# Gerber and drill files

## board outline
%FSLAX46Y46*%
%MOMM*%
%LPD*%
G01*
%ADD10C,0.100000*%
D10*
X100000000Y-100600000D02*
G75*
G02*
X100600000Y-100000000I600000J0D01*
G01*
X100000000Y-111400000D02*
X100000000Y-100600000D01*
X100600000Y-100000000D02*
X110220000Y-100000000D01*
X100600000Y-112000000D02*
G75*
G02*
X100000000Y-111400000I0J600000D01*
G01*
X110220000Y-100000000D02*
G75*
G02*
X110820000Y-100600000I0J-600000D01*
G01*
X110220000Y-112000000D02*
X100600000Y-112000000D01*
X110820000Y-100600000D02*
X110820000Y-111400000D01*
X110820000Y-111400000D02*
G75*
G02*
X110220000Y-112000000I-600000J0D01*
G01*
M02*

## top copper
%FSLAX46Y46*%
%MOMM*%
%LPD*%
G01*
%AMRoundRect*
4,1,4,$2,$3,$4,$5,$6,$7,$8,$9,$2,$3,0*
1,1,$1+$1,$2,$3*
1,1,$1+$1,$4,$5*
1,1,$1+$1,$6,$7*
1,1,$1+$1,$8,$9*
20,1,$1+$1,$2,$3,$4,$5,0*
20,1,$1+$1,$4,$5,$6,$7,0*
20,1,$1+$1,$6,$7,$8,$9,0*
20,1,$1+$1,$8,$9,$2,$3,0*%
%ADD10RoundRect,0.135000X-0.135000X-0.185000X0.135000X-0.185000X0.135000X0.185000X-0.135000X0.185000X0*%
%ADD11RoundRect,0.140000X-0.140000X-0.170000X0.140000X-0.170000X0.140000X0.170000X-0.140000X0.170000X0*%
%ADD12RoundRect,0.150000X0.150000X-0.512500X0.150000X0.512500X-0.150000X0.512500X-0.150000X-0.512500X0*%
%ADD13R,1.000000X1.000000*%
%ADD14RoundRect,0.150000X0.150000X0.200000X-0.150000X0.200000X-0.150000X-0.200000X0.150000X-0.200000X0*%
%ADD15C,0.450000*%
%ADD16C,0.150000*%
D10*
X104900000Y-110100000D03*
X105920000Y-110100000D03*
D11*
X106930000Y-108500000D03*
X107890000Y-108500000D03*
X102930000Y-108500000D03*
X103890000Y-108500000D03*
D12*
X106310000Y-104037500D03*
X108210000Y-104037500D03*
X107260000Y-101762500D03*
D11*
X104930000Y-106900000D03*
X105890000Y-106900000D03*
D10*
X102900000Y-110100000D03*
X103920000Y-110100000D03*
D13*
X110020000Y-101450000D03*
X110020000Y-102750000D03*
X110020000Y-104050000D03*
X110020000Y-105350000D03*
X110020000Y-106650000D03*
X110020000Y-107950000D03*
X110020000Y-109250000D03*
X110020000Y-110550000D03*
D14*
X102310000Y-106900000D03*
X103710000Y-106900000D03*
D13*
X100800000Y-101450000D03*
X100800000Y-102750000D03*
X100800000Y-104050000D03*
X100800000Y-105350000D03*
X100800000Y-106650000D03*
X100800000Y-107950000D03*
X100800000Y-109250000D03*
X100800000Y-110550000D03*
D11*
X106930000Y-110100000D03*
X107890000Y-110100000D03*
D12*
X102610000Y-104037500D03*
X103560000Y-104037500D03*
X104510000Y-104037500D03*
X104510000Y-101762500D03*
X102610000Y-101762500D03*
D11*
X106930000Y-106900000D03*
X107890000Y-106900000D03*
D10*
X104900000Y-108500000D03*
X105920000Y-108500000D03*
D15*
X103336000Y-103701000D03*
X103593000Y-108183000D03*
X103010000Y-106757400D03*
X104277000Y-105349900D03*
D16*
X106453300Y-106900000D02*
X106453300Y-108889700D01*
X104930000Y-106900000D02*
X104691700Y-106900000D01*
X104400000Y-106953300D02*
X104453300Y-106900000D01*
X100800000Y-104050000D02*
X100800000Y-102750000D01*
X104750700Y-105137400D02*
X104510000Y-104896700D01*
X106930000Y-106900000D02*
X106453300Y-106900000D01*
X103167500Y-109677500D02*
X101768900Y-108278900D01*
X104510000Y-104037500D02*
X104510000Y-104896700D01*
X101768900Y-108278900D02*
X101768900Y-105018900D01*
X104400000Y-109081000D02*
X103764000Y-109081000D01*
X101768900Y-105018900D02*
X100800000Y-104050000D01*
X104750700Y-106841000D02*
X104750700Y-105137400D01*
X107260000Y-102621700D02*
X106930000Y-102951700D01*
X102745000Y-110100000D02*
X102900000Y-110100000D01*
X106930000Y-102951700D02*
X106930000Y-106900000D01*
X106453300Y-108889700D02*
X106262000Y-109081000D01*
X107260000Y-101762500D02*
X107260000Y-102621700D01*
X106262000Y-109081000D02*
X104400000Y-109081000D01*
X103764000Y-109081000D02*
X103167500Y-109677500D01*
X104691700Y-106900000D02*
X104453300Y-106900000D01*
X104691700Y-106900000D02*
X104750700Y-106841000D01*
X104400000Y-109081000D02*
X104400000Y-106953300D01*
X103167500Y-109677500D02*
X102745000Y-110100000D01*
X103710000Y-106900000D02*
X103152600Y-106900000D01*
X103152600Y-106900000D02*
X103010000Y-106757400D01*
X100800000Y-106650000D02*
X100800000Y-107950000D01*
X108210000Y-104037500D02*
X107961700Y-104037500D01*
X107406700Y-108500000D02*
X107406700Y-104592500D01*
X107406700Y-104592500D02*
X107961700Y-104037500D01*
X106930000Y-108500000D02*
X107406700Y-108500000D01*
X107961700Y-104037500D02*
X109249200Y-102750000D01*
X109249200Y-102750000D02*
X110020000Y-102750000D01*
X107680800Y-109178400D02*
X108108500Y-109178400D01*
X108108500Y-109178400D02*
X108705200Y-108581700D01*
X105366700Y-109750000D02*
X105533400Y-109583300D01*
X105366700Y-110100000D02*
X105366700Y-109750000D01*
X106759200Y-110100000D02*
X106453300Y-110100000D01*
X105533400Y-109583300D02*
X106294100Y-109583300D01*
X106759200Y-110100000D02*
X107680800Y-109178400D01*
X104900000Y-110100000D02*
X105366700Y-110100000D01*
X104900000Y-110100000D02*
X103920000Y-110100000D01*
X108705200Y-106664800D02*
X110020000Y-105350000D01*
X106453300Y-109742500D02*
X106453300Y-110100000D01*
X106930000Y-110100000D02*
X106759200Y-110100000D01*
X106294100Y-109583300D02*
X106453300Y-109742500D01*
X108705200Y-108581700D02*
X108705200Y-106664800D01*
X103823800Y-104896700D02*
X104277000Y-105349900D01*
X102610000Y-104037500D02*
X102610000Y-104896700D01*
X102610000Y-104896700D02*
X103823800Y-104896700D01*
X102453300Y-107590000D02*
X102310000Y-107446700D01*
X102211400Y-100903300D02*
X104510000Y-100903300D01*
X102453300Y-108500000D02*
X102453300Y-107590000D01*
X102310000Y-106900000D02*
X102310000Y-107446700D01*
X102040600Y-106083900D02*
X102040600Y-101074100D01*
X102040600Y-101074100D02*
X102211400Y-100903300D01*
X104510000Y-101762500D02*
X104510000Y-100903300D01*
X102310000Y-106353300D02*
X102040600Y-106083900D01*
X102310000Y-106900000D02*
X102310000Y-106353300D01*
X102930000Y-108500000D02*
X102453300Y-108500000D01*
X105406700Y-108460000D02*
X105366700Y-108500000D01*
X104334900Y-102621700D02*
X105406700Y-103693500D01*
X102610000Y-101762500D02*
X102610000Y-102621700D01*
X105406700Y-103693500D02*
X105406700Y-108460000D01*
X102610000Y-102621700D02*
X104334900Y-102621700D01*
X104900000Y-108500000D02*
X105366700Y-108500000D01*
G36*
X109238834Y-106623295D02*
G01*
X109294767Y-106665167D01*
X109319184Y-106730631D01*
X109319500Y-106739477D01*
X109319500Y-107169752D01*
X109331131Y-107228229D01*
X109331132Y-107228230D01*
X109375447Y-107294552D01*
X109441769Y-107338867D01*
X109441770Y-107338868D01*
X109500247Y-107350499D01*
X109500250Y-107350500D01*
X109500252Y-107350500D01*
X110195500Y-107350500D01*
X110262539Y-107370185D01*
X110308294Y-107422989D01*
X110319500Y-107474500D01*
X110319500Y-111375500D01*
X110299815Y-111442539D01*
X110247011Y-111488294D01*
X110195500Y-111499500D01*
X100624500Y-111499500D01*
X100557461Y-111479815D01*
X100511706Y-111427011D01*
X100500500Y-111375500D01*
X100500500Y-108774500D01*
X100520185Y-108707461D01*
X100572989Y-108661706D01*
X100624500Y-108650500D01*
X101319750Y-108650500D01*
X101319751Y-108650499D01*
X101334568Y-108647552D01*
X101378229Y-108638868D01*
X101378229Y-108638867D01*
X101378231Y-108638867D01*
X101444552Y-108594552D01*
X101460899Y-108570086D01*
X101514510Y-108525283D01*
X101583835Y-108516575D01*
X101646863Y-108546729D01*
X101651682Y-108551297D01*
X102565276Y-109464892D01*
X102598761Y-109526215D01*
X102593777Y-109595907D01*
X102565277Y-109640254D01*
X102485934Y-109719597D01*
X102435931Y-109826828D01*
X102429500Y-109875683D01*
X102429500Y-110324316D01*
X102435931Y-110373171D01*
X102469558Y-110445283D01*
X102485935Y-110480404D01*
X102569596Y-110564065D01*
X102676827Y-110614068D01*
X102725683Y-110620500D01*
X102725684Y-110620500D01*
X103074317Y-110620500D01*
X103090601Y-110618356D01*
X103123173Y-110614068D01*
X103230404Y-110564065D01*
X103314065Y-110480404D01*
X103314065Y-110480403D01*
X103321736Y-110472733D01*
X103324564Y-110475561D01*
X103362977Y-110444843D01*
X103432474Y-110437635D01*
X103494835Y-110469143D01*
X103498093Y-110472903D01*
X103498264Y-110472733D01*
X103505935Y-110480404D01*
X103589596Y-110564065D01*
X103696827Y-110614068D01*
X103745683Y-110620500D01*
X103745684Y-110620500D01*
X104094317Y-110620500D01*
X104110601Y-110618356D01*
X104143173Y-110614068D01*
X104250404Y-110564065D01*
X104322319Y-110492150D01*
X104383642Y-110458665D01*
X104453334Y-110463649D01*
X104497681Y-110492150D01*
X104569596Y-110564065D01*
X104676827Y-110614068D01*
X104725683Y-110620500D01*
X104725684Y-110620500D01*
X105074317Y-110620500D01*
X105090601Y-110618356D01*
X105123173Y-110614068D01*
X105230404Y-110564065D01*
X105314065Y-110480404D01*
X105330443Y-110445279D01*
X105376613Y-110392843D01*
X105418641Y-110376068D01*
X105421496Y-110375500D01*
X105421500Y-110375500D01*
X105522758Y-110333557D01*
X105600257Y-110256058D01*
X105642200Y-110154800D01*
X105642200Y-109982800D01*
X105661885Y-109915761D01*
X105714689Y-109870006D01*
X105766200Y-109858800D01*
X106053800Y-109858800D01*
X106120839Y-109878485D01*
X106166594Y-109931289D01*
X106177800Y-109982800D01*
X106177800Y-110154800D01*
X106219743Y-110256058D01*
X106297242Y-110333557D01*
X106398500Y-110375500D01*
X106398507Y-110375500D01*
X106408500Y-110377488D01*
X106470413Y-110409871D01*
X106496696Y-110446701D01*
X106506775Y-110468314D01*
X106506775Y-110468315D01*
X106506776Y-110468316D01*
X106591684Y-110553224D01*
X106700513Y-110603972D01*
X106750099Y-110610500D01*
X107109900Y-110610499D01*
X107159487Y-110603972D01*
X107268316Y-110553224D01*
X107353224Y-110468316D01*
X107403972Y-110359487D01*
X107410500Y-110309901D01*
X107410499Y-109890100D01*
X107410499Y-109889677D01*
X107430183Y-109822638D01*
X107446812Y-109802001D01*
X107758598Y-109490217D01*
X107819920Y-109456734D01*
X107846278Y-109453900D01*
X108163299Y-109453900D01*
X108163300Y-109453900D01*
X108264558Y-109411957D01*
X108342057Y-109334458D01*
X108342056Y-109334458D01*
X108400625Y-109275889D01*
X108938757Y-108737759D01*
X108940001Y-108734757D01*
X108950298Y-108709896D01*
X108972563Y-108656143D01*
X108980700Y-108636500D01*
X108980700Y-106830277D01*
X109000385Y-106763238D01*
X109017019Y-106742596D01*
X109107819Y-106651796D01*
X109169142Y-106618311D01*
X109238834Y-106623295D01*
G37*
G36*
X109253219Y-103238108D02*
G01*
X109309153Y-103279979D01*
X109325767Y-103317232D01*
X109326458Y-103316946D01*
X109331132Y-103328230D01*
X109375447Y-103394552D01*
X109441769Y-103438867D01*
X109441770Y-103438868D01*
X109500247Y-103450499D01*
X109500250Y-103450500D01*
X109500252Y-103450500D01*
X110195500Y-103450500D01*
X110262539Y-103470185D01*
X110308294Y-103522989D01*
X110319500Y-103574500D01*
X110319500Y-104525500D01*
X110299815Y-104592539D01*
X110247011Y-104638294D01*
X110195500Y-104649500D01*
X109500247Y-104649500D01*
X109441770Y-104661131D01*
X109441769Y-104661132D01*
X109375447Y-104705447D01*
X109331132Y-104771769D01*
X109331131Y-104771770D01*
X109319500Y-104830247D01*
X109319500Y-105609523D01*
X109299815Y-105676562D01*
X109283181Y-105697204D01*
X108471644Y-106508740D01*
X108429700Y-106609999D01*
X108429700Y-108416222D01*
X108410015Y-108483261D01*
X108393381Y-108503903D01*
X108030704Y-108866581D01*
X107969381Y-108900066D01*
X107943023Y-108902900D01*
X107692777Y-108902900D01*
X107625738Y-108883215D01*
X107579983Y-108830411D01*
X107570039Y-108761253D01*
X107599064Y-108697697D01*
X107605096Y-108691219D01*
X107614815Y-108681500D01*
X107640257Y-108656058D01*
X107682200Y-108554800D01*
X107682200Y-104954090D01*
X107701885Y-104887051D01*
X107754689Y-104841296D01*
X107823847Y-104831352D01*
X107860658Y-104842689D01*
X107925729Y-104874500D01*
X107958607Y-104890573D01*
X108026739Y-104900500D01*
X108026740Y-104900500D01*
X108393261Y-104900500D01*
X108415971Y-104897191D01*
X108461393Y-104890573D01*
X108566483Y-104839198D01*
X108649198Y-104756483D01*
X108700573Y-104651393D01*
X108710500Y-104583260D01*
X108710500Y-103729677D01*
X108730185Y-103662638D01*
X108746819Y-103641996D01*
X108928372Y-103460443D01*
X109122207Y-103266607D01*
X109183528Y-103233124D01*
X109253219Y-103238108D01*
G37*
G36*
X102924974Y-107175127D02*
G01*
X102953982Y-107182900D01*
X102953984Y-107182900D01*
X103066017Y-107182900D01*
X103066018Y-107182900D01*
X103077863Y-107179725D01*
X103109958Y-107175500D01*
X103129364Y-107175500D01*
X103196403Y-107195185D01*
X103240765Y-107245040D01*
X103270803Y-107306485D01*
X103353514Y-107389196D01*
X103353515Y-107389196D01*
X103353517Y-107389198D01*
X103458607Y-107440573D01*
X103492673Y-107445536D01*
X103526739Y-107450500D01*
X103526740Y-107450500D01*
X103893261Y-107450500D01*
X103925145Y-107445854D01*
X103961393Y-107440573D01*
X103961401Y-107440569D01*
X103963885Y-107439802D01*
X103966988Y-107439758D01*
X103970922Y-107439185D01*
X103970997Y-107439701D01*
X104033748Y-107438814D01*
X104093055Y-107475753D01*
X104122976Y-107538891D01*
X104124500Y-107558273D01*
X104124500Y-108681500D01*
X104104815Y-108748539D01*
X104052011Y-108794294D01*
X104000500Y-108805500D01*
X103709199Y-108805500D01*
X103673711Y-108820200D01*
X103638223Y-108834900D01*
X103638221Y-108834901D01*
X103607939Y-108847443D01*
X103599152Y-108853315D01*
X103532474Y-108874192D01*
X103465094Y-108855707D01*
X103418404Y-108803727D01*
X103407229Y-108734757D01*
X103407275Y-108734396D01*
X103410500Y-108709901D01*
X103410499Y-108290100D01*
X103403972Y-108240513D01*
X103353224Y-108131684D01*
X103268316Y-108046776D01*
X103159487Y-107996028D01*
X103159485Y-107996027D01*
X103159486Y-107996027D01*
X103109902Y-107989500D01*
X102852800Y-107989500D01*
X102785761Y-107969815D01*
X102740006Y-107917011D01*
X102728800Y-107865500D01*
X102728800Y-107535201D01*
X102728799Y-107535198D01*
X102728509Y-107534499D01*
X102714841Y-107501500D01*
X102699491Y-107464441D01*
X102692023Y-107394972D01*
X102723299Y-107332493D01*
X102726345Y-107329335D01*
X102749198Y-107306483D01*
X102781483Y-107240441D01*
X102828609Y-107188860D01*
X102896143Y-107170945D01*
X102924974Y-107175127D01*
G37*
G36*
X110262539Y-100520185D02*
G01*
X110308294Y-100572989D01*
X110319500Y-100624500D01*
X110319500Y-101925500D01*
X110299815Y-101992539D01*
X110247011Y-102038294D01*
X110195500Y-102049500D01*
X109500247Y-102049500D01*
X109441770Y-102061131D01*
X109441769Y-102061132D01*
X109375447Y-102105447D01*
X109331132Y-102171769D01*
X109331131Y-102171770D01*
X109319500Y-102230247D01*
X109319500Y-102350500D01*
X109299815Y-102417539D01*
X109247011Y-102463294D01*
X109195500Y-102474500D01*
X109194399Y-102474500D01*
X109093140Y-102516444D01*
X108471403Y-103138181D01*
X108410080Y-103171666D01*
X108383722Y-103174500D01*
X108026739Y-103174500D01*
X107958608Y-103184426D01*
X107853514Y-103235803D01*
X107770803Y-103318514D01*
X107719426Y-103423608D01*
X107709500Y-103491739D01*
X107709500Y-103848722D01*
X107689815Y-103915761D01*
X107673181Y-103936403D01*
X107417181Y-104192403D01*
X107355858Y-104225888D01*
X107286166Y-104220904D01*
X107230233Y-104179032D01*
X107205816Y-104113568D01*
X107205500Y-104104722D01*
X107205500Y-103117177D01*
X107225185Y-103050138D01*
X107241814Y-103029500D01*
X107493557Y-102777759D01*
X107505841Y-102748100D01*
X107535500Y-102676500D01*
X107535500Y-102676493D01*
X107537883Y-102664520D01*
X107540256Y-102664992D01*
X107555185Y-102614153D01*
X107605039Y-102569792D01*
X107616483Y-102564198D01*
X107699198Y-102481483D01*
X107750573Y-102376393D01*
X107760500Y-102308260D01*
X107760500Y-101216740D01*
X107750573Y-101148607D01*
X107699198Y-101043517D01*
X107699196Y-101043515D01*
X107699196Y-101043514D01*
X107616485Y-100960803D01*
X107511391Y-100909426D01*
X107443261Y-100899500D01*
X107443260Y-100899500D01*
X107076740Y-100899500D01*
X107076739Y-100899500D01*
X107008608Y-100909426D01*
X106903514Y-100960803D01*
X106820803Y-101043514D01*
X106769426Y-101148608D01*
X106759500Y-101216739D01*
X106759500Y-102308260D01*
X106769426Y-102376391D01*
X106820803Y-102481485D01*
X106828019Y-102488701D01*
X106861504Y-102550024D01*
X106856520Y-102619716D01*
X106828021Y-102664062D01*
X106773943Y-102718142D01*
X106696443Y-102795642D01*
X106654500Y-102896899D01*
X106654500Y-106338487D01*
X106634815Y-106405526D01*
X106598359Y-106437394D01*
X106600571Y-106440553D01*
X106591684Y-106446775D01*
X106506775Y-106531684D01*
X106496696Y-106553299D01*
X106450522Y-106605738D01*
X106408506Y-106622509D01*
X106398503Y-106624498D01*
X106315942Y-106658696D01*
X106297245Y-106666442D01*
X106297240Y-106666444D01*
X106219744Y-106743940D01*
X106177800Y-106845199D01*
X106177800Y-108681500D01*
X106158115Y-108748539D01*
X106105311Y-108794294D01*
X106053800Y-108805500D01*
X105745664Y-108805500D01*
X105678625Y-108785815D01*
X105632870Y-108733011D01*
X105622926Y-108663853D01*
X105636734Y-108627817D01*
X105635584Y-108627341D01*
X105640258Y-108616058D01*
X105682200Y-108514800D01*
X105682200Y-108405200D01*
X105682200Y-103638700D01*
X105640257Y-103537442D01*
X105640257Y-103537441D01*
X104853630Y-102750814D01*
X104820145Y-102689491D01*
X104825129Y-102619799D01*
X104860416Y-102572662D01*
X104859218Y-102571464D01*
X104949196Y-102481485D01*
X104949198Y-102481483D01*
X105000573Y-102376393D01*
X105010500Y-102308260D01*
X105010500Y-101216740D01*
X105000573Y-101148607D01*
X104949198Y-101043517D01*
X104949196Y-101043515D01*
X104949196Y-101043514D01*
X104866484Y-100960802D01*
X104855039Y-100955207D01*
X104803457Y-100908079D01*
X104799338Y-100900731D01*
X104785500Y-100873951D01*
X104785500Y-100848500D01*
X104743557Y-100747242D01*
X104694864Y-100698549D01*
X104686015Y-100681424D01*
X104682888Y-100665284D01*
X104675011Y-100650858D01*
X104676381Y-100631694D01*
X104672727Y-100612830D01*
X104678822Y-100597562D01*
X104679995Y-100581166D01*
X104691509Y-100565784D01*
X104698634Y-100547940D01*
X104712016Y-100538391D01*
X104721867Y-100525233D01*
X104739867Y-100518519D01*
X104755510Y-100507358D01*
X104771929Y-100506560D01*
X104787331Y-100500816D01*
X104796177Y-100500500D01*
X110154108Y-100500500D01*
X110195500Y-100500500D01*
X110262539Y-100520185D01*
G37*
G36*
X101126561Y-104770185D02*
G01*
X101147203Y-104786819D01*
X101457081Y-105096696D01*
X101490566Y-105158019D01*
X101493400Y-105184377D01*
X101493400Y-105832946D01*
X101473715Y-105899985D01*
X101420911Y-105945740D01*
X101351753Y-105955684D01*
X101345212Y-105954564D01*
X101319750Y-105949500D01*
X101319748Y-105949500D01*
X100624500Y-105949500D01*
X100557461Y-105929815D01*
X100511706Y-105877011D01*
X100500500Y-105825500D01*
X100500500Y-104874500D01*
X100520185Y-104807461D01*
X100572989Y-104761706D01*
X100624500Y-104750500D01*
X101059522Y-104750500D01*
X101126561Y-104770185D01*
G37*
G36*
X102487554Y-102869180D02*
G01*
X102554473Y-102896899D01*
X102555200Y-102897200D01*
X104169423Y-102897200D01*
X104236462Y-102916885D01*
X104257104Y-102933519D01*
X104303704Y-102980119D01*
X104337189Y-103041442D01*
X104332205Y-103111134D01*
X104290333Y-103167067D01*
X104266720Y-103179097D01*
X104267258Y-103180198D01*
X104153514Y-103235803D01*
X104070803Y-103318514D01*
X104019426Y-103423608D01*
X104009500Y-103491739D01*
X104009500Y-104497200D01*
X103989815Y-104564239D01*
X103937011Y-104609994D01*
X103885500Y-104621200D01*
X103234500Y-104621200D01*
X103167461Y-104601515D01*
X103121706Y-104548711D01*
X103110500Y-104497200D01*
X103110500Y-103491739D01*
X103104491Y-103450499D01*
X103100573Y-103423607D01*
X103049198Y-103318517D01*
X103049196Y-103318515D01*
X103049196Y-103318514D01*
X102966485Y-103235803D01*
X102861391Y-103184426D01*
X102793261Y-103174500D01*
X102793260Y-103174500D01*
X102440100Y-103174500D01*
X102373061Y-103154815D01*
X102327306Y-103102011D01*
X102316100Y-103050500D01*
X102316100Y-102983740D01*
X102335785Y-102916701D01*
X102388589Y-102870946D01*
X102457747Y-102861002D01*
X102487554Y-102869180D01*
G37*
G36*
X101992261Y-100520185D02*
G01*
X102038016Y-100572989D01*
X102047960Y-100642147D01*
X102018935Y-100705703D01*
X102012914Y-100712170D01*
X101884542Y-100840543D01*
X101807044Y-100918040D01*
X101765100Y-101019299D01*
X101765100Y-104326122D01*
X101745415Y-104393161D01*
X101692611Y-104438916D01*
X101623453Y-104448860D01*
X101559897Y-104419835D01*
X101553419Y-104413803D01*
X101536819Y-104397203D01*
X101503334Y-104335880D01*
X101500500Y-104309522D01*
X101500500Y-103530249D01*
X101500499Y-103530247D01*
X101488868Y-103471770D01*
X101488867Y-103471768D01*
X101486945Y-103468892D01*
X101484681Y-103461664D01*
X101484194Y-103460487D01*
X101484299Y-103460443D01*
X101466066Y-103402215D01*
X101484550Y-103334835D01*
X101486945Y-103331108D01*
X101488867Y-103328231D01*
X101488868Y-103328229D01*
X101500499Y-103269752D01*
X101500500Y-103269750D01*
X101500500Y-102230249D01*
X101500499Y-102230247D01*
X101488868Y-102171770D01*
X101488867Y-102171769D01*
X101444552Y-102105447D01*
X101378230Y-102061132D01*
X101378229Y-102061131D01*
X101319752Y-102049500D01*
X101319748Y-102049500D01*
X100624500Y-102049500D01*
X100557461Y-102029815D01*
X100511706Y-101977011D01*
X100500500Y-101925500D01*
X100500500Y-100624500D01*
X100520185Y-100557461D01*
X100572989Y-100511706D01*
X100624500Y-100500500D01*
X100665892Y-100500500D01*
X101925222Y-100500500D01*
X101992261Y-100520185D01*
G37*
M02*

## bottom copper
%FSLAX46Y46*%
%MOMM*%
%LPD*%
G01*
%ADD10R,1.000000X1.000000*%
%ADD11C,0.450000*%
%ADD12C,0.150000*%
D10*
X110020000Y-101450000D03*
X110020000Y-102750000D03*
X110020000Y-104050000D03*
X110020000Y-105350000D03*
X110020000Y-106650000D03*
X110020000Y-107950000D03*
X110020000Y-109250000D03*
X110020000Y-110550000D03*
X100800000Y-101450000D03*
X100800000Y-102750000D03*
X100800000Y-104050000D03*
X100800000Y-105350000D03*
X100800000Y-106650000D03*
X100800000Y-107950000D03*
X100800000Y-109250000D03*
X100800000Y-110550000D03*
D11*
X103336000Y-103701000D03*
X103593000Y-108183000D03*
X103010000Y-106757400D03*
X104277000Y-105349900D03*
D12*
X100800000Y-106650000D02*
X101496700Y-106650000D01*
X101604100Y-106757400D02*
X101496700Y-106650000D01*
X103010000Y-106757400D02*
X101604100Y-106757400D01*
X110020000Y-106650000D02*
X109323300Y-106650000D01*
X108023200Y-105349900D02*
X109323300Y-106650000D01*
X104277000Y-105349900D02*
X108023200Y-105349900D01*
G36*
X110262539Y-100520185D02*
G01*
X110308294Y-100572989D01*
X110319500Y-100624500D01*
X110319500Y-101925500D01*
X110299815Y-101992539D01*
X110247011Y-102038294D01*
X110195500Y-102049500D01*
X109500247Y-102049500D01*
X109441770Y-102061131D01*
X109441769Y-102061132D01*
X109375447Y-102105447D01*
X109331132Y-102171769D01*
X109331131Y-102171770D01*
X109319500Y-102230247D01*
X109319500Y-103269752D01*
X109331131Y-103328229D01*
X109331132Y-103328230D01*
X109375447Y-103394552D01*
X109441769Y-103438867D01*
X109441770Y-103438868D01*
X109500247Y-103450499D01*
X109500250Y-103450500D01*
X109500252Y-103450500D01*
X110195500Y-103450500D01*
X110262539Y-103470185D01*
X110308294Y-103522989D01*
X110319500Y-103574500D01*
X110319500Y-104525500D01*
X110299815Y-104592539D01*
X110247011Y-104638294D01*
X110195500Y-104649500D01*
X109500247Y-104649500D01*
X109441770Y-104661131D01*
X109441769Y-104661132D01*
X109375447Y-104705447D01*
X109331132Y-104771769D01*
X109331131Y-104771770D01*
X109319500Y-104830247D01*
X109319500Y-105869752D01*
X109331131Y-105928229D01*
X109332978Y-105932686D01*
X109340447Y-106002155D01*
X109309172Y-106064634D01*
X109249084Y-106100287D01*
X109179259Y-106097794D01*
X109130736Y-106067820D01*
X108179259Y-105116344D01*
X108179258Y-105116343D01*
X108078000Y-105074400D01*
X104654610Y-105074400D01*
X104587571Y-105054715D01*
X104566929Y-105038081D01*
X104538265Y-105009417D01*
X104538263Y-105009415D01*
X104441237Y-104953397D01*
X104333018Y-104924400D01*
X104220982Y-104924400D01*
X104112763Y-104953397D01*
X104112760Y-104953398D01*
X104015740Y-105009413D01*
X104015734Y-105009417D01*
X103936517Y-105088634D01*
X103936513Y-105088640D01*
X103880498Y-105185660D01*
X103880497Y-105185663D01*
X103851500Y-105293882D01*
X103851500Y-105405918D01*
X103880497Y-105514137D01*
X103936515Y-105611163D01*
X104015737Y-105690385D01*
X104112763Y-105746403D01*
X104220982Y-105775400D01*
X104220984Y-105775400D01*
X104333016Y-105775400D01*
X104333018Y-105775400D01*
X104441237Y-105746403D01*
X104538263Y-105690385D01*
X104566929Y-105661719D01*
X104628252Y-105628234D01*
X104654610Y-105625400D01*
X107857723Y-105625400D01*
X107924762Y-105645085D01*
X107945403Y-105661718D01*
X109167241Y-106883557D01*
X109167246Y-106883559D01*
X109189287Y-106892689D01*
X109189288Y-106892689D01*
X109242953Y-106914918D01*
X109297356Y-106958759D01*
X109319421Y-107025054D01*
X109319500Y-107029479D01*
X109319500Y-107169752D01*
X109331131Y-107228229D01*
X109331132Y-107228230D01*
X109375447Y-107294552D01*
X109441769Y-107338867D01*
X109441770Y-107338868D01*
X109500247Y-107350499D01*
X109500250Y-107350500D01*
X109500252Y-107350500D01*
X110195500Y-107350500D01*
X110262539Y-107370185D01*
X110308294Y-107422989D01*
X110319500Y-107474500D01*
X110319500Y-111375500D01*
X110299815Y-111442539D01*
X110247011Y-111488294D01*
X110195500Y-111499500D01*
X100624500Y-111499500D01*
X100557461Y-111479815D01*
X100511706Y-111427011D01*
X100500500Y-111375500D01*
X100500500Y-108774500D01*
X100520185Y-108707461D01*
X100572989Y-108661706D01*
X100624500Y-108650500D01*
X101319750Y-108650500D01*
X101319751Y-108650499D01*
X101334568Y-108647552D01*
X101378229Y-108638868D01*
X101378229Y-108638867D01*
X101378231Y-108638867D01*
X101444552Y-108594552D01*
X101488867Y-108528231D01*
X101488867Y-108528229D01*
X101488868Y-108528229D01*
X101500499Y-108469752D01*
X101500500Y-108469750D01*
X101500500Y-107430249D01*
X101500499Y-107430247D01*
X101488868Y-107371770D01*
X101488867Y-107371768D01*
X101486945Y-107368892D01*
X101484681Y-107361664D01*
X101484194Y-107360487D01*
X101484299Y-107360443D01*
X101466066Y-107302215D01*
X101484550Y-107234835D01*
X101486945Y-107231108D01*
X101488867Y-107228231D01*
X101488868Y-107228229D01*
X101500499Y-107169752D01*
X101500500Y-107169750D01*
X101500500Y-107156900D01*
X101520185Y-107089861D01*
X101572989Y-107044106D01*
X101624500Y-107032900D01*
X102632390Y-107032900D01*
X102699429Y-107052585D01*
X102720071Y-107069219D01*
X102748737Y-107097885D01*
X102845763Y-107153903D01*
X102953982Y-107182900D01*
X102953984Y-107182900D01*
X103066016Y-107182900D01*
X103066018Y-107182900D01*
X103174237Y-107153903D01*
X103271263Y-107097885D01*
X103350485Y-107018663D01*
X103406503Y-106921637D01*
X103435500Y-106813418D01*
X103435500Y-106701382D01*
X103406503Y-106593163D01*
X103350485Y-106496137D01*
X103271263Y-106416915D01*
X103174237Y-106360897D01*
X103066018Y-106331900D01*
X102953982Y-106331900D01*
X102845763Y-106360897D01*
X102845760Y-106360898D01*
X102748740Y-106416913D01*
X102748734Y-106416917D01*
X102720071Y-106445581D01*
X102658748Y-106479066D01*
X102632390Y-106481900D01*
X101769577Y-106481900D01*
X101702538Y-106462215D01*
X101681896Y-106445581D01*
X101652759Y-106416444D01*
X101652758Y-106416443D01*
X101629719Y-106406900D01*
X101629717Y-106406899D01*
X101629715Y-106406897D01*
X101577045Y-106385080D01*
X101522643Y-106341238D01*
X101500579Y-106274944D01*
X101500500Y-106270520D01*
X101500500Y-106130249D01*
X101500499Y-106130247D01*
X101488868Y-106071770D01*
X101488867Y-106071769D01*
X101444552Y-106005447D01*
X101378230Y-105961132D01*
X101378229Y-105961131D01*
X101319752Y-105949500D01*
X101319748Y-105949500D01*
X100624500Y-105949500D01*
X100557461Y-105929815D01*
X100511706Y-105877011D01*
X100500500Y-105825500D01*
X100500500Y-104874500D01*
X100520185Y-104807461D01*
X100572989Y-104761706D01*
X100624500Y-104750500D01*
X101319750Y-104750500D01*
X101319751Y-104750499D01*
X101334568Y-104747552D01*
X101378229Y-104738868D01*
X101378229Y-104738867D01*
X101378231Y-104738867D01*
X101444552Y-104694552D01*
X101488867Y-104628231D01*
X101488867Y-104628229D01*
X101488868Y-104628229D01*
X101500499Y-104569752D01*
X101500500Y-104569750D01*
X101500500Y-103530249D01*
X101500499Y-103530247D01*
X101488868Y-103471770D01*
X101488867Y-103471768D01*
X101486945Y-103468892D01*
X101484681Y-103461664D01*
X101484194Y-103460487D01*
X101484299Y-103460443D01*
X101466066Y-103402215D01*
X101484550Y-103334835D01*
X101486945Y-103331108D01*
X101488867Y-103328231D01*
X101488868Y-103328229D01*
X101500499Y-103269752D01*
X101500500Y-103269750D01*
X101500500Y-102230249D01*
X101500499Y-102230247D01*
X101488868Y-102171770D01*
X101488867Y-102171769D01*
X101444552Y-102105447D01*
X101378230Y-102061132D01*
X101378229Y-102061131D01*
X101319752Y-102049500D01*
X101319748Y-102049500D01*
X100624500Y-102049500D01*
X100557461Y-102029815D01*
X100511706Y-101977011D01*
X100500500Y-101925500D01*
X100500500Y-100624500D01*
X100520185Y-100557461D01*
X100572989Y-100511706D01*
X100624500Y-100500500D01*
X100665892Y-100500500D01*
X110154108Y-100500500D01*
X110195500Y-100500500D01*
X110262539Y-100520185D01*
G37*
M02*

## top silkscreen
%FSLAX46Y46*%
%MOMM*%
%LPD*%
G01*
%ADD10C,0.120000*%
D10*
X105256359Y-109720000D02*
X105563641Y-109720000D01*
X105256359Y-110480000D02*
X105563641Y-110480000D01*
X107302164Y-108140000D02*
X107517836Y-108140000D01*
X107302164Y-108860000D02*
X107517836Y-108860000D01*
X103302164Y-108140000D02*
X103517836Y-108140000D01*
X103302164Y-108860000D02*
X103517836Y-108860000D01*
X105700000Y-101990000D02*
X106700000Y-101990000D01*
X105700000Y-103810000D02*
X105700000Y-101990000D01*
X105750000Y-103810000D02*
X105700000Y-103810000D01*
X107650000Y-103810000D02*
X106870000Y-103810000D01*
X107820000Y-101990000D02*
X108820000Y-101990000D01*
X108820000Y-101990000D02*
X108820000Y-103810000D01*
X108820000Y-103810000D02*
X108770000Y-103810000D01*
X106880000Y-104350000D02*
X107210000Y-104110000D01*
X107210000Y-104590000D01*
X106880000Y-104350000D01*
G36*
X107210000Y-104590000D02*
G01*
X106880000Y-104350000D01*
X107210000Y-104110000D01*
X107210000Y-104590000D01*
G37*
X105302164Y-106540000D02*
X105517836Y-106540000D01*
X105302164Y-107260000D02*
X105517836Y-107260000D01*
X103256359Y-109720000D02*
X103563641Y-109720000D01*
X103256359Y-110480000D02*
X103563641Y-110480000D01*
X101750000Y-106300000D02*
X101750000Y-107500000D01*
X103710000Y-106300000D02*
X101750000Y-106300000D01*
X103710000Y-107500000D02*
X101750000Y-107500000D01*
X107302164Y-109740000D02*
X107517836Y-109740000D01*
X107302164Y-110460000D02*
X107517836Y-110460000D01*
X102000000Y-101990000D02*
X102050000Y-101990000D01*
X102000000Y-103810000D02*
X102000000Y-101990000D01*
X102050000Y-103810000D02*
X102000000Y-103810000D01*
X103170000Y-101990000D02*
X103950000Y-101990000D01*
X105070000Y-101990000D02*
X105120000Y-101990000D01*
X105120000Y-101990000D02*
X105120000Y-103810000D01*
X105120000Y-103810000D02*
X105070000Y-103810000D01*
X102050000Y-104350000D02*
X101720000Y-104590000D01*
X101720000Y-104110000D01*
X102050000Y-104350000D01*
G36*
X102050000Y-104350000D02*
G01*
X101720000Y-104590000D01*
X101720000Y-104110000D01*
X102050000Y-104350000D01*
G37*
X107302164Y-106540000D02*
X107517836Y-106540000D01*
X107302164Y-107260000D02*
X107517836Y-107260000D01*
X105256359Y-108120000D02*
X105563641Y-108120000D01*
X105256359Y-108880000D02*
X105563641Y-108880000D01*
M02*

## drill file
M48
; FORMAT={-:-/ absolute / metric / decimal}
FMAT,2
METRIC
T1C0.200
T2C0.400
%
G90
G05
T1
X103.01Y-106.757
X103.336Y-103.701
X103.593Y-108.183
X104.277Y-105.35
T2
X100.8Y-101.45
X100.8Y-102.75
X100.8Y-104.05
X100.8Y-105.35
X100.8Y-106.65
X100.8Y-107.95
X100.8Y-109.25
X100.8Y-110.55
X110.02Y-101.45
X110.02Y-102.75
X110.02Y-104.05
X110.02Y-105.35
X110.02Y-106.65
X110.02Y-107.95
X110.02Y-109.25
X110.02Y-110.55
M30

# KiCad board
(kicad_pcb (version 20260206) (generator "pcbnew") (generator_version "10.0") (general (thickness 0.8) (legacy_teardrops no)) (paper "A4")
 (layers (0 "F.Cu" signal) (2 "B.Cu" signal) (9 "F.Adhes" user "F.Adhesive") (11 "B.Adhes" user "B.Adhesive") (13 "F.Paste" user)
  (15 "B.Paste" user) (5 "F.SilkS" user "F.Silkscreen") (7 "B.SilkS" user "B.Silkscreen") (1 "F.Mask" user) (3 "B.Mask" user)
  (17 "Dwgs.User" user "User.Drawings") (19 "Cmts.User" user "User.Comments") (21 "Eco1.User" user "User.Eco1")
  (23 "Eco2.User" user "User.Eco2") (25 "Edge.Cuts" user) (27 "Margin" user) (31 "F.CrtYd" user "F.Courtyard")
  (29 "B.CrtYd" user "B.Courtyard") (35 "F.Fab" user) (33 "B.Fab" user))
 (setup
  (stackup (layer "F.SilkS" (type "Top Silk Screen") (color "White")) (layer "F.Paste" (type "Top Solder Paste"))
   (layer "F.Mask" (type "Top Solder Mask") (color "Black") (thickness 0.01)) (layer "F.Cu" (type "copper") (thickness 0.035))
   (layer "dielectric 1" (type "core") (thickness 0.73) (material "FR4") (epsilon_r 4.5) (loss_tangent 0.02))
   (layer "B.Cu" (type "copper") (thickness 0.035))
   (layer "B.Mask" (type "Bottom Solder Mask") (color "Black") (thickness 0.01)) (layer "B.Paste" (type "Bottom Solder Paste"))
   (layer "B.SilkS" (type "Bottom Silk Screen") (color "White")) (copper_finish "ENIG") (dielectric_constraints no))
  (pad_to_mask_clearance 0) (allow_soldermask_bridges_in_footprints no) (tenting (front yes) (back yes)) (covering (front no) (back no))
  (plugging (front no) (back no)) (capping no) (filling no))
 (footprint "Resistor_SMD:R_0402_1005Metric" (layer "F.Cu") (at 105.41 110.1)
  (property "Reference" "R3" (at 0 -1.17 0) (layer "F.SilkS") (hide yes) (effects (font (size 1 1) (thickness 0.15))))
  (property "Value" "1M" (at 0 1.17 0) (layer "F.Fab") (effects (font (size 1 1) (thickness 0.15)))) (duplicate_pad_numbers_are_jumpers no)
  (fp_line (start -0.153641 -0.38) (end 0.153641 -0.38) (stroke (width 0.12) (type solid)) (layer "F.SilkS"))
  (fp_line (start -0.153641 0.38) (end 0.153641 0.38) (stroke (width 0.12) (type solid)) (layer "F.SilkS"))
  (pad "1" smd roundrect (at -0.51 0) (size 0.54 0.64) (layers "F.Cu" "F.Mask" "F.Paste") (roundrect_rratio 0.25) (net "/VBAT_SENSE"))
  (pad "2" smd roundrect (at 0.51 0) (size 0.54 0.64) (layers "F.Cu" "F.Mask" "F.Paste") (roundrect_rratio 0.25) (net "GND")))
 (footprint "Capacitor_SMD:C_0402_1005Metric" (layer "F.Cu") (at 107.41 108.5)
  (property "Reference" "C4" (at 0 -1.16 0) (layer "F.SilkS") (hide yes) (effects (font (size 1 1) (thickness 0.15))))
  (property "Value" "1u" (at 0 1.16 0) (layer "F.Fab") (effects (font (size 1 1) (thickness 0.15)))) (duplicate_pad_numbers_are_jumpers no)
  (fp_line (start -0.107836 -0.36) (end 0.107836 -0.36) (stroke (width 0.12) (type solid)) (layer "F.SilkS"))
  (fp_line (start -0.107836 0.36) (end 0.107836 0.36) (stroke (width 0.12) (type solid)) (layer "F.SilkS"))
  (pad "1" smd roundrect (at -0.48 0) (size 0.56 0.62) (layers "F.Cu" "F.Mask" "F.Paste") (roundrect_rratio 0.25) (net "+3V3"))
  (pad "2" smd roundrect (at 0.48 0) (size 0.56 0.62) (layers "F.Cu" "F.Mask" "F.Paste") (roundrect_rratio 0.25) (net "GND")))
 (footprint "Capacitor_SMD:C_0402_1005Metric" (layer "F.Cu") (at 103.41 108.5)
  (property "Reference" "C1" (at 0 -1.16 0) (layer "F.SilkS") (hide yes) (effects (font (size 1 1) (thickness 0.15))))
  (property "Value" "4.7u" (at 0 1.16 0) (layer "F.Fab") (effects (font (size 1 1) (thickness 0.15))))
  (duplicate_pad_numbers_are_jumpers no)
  (fp_line (start -0.107836 -0.36) (end 0.107836 -0.36) (stroke (width 0.12) (type solid)) (layer "F.SilkS"))
  (fp_line (start -0.107836 0.36) (end 0.107836 0.36) (stroke (width 0.12) (type solid)) (layer "F.SilkS"))
  (pad "1" smd roundrect (at -0.48 0) (size 0.56 0.62) (layers "F.Cu" "F.Mask" "F.Paste") (roundrect_rratio 0.25) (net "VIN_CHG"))
  (pad "2" smd roundrect (at 0.48 0) (size 0.56 0.62) (layers "F.Cu" "F.Mask" "F.Paste") (roundrect_rratio 0.25) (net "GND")))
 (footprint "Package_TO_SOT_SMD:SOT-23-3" (layer "F.Cu") (at 107.26 102.9 90)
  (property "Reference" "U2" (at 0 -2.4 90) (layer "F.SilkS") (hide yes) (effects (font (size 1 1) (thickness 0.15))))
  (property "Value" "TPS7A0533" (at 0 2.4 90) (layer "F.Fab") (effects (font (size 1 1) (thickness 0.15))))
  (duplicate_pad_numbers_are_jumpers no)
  (fp_line (start 0.91 -1.56) (end 0.91 -0.56) (stroke (width 0.12) (type solid)) (layer "F.SilkS"))
  (fp_line (start -0.91 -1.56) (end 0.91 -1.56) (stroke (width 0.12) (type solid)) (layer "F.SilkS"))
  (fp_line (start -0.91 -1.51) (end -0.91 -1.56) (stroke (width 0.12) (type solid)) (layer "F.SilkS"))
  (fp_line (start -0.91 0.39) (end -0.91 -0.39) (stroke (width 0.12) (type solid)) (layer "F.SilkS"))
  (fp_line (start 0.91 0.56) (end 0.91 1.56) (stroke (width 0.12) (type solid)) (layer "F.SilkS"))
  (fp_line (start 0.91 1.56) (end -0.91 1.56) (stroke (width 0.12) (type solid)) (layer "F.SilkS"))
  (fp_line (start -0.91 1.56) (end -0.91 1.51) (stroke (width 0.12) (type solid)) (layer "F.SilkS"))
  (fp_poly (pts (xy -1.45 -0.38) (xy -1.21 -0.05) (xy -1.69 -0.05)) (stroke (width 0.12) (type solid)) (fill yes) (layer "F.SilkS"))
  (pad "1" smd roundrect (at -1.1375 -0.95 90) (size 1.325 0.6) (layers "F.Cu" "F.Mask" "F.Paste") (roundrect_rratio 0.25) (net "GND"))
  (pad "2" smd roundrect (at -1.1375 0.95 90) (size 1.325 0.6) (layers "F.Cu" "F.Mask" "F.Paste") (roundrect_rratio 0.25) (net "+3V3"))
  (pad "3" smd roundrect (at 1.1375 0 90) (size 1.325 0.6) (layers "F.Cu" "F.Mask" "F.Paste") (roundrect_rratio 0.25) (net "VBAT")))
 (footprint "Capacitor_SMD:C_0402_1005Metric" (layer "F.Cu") (at 105.41 106.9)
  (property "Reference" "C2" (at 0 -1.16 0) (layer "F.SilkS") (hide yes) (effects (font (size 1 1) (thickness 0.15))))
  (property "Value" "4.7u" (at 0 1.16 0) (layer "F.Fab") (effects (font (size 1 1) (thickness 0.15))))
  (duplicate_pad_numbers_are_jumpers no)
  (fp_line (start -0.107836 -0.36) (end 0.107836 -0.36) (stroke (width 0.12) (type solid)) (layer "F.SilkS"))
  (fp_line (start -0.107836 0.36) (end 0.107836 0.36) (stroke (width 0.12) (type solid)) (layer "F.SilkS"))
  (pad "1" smd roundrect (at -0.48 0) (size 0.56 0.62) (layers "F.Cu" "F.Mask" "F.Paste") (roundrect_rratio 0.25) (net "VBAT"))
  (pad "2" smd roundrect (at 0.48 0) (size 0.56 0.62) (layers "F.Cu" "F.Mask" "F.Paste") (roundrect_rratio 0.25) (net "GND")))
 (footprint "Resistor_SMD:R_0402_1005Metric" (layer "F.Cu") (at 103.41 110.1)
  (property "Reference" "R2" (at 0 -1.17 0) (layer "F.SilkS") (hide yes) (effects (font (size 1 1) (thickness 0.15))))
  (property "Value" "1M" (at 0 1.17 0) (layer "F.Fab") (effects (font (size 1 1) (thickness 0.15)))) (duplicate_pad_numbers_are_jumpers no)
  (fp_line (start -0.153641 -0.38) (end 0.153641 -0.38) (stroke (width 0.12) (type solid)) (layer "F.SilkS"))
  (fp_line (start -0.153641 0.38) (end 0.153641 0.38) (stroke (width 0.12) (type solid)) (layer "F.SilkS"))
  (pad "1" smd roundrect (at -0.51 0) (size 0.54 0.64) (layers "F.Cu" "F.Mask" "F.Paste") (roundrect_rratio 0.25) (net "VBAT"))
  (pad "2" smd roundrect (at 0.51 0) (size 0.54 0.64) (layers "F.Cu" "F.Mask" "F.Paste") (roundrect_rratio 0.25) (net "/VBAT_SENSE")))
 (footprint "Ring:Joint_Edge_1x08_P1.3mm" (layer "F.Cu") (at 110.02 106)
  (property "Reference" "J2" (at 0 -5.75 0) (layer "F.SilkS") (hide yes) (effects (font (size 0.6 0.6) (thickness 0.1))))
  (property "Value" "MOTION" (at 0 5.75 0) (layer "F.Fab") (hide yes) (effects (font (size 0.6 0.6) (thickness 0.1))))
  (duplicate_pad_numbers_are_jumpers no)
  (pad "1" thru_hole rect (at 0 -4.55) (size 1 1) (drill 0.4) (layers "*.Cu" "*.Mask") (remove_unused_layers no) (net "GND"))
  (pad "2" thru_hole rect (at 0 -3.25) (size 1 1) (drill 0.4) (layers "*.Cu" "*.Mask") (remove_unused_layers no) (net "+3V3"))
  (pad "3" thru_hole rect (at 0 -1.95) (size 1 1) (drill 0.4) (layers "*.Cu" "*.Mask") (remove_unused_layers no) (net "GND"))
  (pad "4" thru_hole rect (at 0 -0.65) (size 1 1) (drill 0.4) (layers "*.Cu" "*.Mask") (remove_unused_layers no) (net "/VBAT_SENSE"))
  (pad "5" thru_hole rect (at 0 0.65) (size 1 1) (drill 0.4) (layers "*.Cu" "*.Mask") (remove_unused_layers no) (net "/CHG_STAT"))
  (pad "6" thru_hole rect (at 0 1.95) (size 1 1) (drill 0.4) (layers "*.Cu" "*.Mask") (remove_unused_layers no) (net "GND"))
  (pad "7" thru_hole rect (at 0 3.25) (size 1 1) (drill 0.4) (layers "*.Cu" "*.Mask") (remove_unused_layers no) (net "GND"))
  (pad "8" thru_hole rect (at 0 4.55) (size 1 1) (drill 0.4) (layers "*.Cu" "*.Mask") (remove_unused_layers no) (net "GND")))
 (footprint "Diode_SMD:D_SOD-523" (layer "F.Cu") (at 103.01 106.9)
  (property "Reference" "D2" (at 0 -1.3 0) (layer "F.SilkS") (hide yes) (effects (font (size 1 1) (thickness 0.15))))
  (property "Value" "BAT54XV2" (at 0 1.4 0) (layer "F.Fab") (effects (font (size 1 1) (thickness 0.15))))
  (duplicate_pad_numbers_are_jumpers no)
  (fp_line (start -1.26 -0.6) (end -1.26 0.6) (stroke (width 0.12) (type solid)) (layer "F.SilkS"))
  (fp_line (start 0.7 -0.6) (end -1.26 -0.6) (stroke (width 0.12) (type solid)) (layer "F.SilkS"))
  (fp_line (start 0.7 0.6) (end -1.26 0.6) (stroke (width 0.12) (type solid)) (layer "F.SilkS"))
  (pad "1" smd roundrect (at -0.7 0 180) (size 0.6 0.7) (layers "F.Cu" "F.Mask" "F.Paste") (roundrect_rratio 0.25) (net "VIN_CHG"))
  (pad "2" smd roundrect (at 0.7 0 180) (size 0.6 0.7) (layers "F.Cu" "F.Mask" "F.Paste") (roundrect_rratio 0.25) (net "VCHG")))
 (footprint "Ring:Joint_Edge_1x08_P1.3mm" (layer "F.Cu") (at 100.8 106)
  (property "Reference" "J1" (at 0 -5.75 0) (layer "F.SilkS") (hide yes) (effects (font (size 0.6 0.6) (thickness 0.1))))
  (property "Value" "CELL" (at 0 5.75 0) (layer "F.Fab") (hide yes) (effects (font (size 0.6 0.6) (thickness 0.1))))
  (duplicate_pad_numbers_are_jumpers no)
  (pad "1" thru_hole rect (at 0 -4.55) (size 1 1) (drill 0.4) (layers "*.Cu" "*.Mask") (remove_unused_layers no) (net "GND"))
  (pad "2" thru_hole rect (at 0 -3.25) (size 1 1) (drill 0.4) (layers "*.Cu" "*.Mask") (remove_unused_layers no) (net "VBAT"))
  (pad "3" thru_hole rect (at 0 -1.95) (size 1 1) (drill 0.4) (layers "*.Cu" "*.Mask") (remove_unused_layers no) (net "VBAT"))
  (pad "4" thru_hole rect (at 0 -0.65) (size 1 1) (drill 0.4) (layers "*.Cu" "*.Mask") (remove_unused_layers no) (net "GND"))
  (pad "5" thru_hole rect (at 0 0.65) (size 1 1) (drill 0.4) (layers "*.Cu" "*.Mask") (remove_unused_layers no) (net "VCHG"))
  (pad "6" thru_hole rect (at 0 1.95) (size 1 1) (drill 0.4) (layers "*.Cu" "*.Mask") (remove_unused_layers no) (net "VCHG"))
  (pad "7" thru_hole rect (at 0 3.25) (size 1 1) (drill 0.4) (layers "*.Cu" "*.Mask") (remove_unused_layers no) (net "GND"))
  (pad "8" thru_hole rect (at 0 4.55) (size 1 1) (drill 0.4) (layers "*.Cu" "*.Mask") (remove_unused_layers no) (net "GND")))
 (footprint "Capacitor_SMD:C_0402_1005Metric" (layer "F.Cu") (at 107.41 110.1)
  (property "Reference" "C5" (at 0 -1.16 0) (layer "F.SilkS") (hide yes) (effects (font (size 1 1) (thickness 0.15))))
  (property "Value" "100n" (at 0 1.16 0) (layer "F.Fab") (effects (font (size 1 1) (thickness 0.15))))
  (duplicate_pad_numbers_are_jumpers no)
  (fp_line (start -0.107836 -0.36) (end 0.107836 -0.36) (stroke (width 0.12) (type solid)) (layer "F.SilkS"))
  (fp_line (start -0.107836 0.36) (end 0.107836 0.36) (stroke (width 0.12) (type solid)) (layer "F.SilkS"))
  (pad "1" smd roundrect (at -0.48 0) (size 0.56 0.62) (layers "F.Cu" "F.Mask" "F.Paste") (roundrect_rratio 0.25) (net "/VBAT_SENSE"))
  (pad "2" smd roundrect (at 0.48 0) (size 0.56 0.62) (layers "F.Cu" "F.Mask" "F.Paste") (roundrect_rratio 0.25) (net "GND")))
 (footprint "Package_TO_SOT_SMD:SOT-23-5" (layer "F.Cu") (at 103.56 102.9 90)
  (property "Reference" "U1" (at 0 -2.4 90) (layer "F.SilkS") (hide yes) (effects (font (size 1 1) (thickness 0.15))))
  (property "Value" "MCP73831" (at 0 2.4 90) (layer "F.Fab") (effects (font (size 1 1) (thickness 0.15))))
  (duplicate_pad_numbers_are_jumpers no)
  (fp_line (start 0.91 -1.56) (end 0.91 -1.51) (stroke (width 0.12) (type solid)) (layer "F.SilkS"))
  (fp_line (start -0.91 -1.56) (end 0.91 -1.56) (stroke (width 0.12) (type solid)) (layer "F.SilkS"))
  (fp_line (start -0.91 -1.51) (end -0.91 -1.56) (stroke (width 0.12) (type solid)) (layer "F.SilkS"))
  (fp_line (start 0.91 -0.39) (end 0.91 0.39) (stroke (width 0.12) (type solid)) (layer "F.SilkS"))
  (fp_line (start 0.91 1.51) (end 0.91 1.56) (stroke (width 0.12) (type solid)) (layer "F.SilkS"))
  (fp_line (start 0.91 1.56) (end -0.91 1.56) (stroke (width 0.12) (type solid)) (layer "F.SilkS"))
  (fp_line (start -0.91 1.56) (end -0.91 1.51) (stroke (width 0.12) (type solid)) (layer "F.SilkS"))
  (fp_poly (pts (xy -1.45 -1.51) (xy -1.69 -1.84) (xy -1.21 -1.84)) (stroke (width 0.12) (type solid)) (fill yes) (layer "F.SilkS"))
  (pad "1" smd roundrect (at -1.1375 -0.95 90) (size 1.325 0.6) (layers "F.Cu" "F.Mask" "F.Paste") (roundrect_rratio 0.25) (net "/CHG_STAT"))
  (pad "2" smd roundrect (at -1.1375 0 90) (size 1.325 0.6) (layers "F.Cu" "F.Mask" "F.Paste") (roundrect_rratio 0.25) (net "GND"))
  (pad "3" smd roundrect (at -1.1375 0.95 90) (size 1.325 0.6) (layers "F.Cu" "F.Mask" "F.Paste") (roundrect_rratio 0.25) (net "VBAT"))
  (pad "4" smd roundrect (at 1.1375 0.95 90) (size 1.325 0.6) (layers "F.Cu" "F.Mask" "F.Paste") (roundrect_rratio 0.25) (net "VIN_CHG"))
  (pad "5" smd roundrect (at 1.1375 -0.95 90) (size 1.325 0.6) (layers "F.Cu" "F.Mask" "F.Paste") (roundrect_rratio 0.25) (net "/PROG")))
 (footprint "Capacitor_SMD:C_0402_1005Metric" (layer "F.Cu") (at 107.41 106.9)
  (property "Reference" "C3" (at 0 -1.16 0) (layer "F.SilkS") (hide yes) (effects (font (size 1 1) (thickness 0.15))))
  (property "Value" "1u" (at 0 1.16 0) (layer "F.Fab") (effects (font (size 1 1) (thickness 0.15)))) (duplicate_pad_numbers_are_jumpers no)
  (fp_line (start -0.107836 -0.36) (end 0.107836 -0.36) (stroke (width 0.12) (type solid)) (layer "F.SilkS"))
  (fp_line (start -0.107836 0.36) (end 0.107836 0.36) (stroke (width 0.12) (type solid)) (layer "F.SilkS"))
  (pad "1" smd roundrect (at -0.48 0) (size 0.56 0.62) (layers "F.Cu" "F.Mask" "F.Paste") (roundrect_rratio 0.25) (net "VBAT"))
  (pad "2" smd roundrect (at 0.48 0) (size 0.56 0.62) (layers "F.Cu" "F.Mask" "F.Paste") (roundrect_rratio 0.25) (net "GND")))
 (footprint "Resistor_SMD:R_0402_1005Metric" (layer "F.Cu") (at 105.41 108.5)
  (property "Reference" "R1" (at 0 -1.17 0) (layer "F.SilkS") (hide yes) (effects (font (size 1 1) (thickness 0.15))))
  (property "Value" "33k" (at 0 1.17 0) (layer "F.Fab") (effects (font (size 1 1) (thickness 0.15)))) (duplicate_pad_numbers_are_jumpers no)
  (fp_line (start -0.153641 -0.38) (end 0.153641 -0.38) (stroke (width 0.12) (type solid)) (layer "F.SilkS"))
  (fp_line (start -0.153641 0.38) (end 0.153641 0.38) (stroke (width 0.12) (type solid)) (layer "F.SilkS"))
  (pad "1" smd roundrect (at -0.51 0) (size 0.54 0.64) (layers "F.Cu" "F.Mask" "F.Paste") (roundrect_rratio 0.25) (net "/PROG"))
  (pad "2" smd roundrect (at 0.51 0) (size 0.54 0.64) (layers "F.Cu" "F.Mask" "F.Paste") (roundrect_rratio 0.25) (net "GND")))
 (gr_arc (start 100 100.6) (mid 100.175736 100.175736) (end 100.6 100) (stroke (width 0.1) (type default)) (layer "Edge.Cuts"))
 (gr_line (start 100 111.4) (end 100 100.6) (stroke (width 0.1) (type default)) (layer "Edge.Cuts"))
 (gr_line (start 100.6 100) (end 110.22 100) (stroke (width 0.1) (type default)) (layer "Edge.Cuts"))
 (gr_arc (start 100.6 112) (mid 100.175736 111.824264) (end 100 111.4) (stroke (width 0.1) (type default)) (layer "Edge.Cuts"))
 (gr_arc (start 110.22 100) (mid 110.644264 100.175736) (end 110.82 100.6) (stroke (width 0.1) (type default)) (layer "Edge.Cuts"))
 (gr_line (start 110.22 112) (end 100.6 112) (stroke (width 0.1) (type default)) (layer "Edge.Cuts"))
 (gr_line (start 110.82 100.6) (end 110.82 111.4) (stroke (width 0.1) (type default)) (layer "Edge.Cuts"))
 (gr_arc (start 110.82 111.4) (mid 110.644264 111.824264) (end 110.22 112) (stroke (width 0.1) (type default)) (layer "Edge.Cuts"))
 (via (at 103.336 103.701) (size 0.45) (drill 0.2) (layers "F.Cu" "B.Cu") (capping no) (covering (front no) (back no))
  (plugging (front no) (back no)) (filling no) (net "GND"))
 (via (at 103.593 108.183) (size 0.45) (drill 0.2) (layers "F.Cu" "B.Cu") (capping no) (covering (front no) (back no))
  (plugging (front no) (back no)) (filling no) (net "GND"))
 (segment (start 106.4533 106.9) (end 106.4533 108.8897) (width 0.15) (layer "F.Cu") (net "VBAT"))
 (segment (start 104.93 106.9) (end 104.6917 106.9) (width 0.15) (layer "F.Cu") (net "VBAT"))
 (segment (start 104.4 106.9533) (end 104.4533 106.9) (width 0.15) (layer "F.Cu") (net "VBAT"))
 (segment (start 100.8 104.05) (end 100.8 102.75) (width 0.15) (layer "F.Cu") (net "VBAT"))
 (segment (start 104.7507 105.1374) (end 104.51 104.8967) (width 0.15) (layer "F.Cu") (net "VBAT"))
 (segment (start 106.93 106.9) (end 106.4533 106.9) (width 0.15) (layer "F.Cu") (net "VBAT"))
 (segment (start 103.1675 109.6775) (end 101.7689 108.2789) (width 0.15) (layer "F.Cu") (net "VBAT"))
 (segment (start 104.51 104.0375) (end 104.51 104.8967) (width 0.15) (layer "F.Cu") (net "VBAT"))
 (segment (start 101.7689 108.2789) (end 101.7689 105.0189) (width 0.15) (layer "F.Cu") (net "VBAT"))
 (segment (start 104.4 109.081) (end 103.764 109.081) (width 0.15) (layer "F.Cu") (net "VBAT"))
 (segment (start 101.7689 105.0189) (end 100.8 104.05) (width 0.15) (layer "F.Cu") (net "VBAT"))
 (segment (start 104.7507 106.841) (end 104.7507 105.1374) (width 0.15) (layer "F.Cu") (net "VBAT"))
 (segment (start 107.26 102.6217) (end 106.93 102.9517) (width 0.15) (layer "F.Cu") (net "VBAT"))
 (segment (start 102.745 110.1) (end 102.9 110.1) (width 0.15) (layer "F.Cu") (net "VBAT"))
 (segment (start 106.93 102.9517) (end 106.93 106.9) (width 0.15) (layer "F.Cu") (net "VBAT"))
 (segment (start 106.4533 108.8897) (end 106.262 109.081) (width 0.15) (layer "F.Cu") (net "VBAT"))
 (segment (start 107.26 101.7625) (end 107.26 102.6217) (width 0.15) (layer "F.Cu") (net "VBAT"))
 (segment (start 106.262 109.081) (end 104.4 109.081) (width 0.15) (layer "F.Cu") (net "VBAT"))
 (segment (start 103.764 109.081) (end 103.1675 109.6775) (width 0.15) (layer "F.Cu") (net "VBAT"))
 (segment (start 104.6917 106.9) (end 104.4533 106.9) (width 0.15) (layer "F.Cu") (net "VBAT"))
 (segment (start 104.6917 106.9) (end 104.7507 106.841) (width 0.15) (layer "F.Cu") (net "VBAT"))
 (segment (start 104.4 109.081) (end 104.4 106.9533) (width 0.15) (layer "F.Cu") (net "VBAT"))
 (segment (start 103.1675 109.6775) (end 102.745 110.1) (width 0.15) (layer "F.Cu") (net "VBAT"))
 (segment (start 103.71 106.9) (end 103.1526 106.9) (width 0.15) (layer "F.Cu") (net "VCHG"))
 (segment (start 103.1526 106.9) (end 103.01 106.7574) (width 0.15) (layer "F.Cu") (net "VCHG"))
 (segment (start 100.8 106.65) (end 100.8 107.95) (width 0.15) (layer "F.Cu") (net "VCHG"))
 (via (at 103.01 106.7574) (size 0.45) (drill 0.2) (layers "F.Cu" "B.Cu") (capping no) (covering (front no) (back no))
  (plugging (front no) (back no)) (filling no) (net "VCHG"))
 (segment (start 100.8 106.65) (end 101.4967 106.65) (width 0.15) (layer "B.Cu") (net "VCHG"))
 (segment (start 101.6041 106.7574) (end 101.4967 106.65) (width 0.15) (layer "B.Cu") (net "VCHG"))
 (segment (start 103.01 106.7574) (end 101.6041 106.7574) (width 0.15) (layer "B.Cu") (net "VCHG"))
 (segment (start 108.21 104.0375) (end 107.9617 104.0375) (width 0.15) (layer "F.Cu") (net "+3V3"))
 (segment (start 107.4067 108.5) (end 107.4067 104.5925) (width 0.15) (layer "F.Cu") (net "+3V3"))
 (segment (start 107.4067 104.5925) (end 107.9617 104.0375) (width 0.15) (layer "F.Cu") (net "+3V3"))
 (segment (start 106.93 108.5) (end 107.4067 108.5) (width 0.15) (layer "F.Cu") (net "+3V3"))
 (segment (start 107.9617 104.0375) (end 109.2492 102.75) (width 0.15) (layer "F.Cu") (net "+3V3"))
 (segment (start 109.2492 102.75) (end 110.02 102.75) (width 0.15) (layer "F.Cu") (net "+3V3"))
 (segment (start 107.6808 109.1784) (end 108.1085 109.1784) (width 0.15) (layer "F.Cu") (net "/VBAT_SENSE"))
 (segment (start 108.1085 109.1784) (end 108.7052 108.5817) (width 0.15) (layer "F.Cu") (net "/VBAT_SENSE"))
 (segment (start 105.3667 109.75) (end 105.5334 109.5833) (width 0.15) (layer "F.Cu") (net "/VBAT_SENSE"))
 (segment (start 105.3667 110.1) (end 105.3667 109.75) (width 0.15) (layer "F.Cu") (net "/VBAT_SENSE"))
 (segment (start 106.7592 110.1) (end 106.4533 110.1) (width 0.15) (layer "F.Cu") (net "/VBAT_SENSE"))
 (segment (start 105.5334 109.5833) (end 106.2941 109.5833) (width 0.15) (layer "F.Cu") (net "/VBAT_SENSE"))
 (segment (start 106.7592 110.1) (end 107.6808 109.1784) (width 0.15) (layer "F.Cu") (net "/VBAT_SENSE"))
 (segment (start 104.9 110.1) (end 105.3667 110.1) (width 0.15) (layer "F.Cu") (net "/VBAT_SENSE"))
 (segment (start 104.9 110.1) (end 103.92 110.1) (width 0.15) (layer "F.Cu") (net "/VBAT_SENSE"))
 (segment (start 108.7052 106.6648) (end 110.02 105.35) (width 0.15) (layer "F.Cu") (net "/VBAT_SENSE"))
 (segment (start 106.4533 109.7425) (end 106.4533 110.1) (width 0.15) (layer "F.Cu") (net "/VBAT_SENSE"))
 (segment (start 106.93 110.1) (end 106.7592 110.1) (width 0.15) (layer "F.Cu") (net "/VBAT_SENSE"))
 (segment (start 106.2941 109.5833) (end 106.4533 109.7425) (width 0.15) (layer "F.Cu") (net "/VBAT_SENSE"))
 (segment (start 108.7052 108.5817) (end 108.7052 106.6648) (width 0.15) (layer "F.Cu") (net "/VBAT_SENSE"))
 (segment (start 103.8238 104.8967) (end 104.277 105.3499) (width 0.15) (layer "F.Cu") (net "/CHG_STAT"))
 (segment (start 102.61 104.0375) (end 102.61 104.8967) (width 0.15) (layer "F.Cu") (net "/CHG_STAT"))
 (segment (start 102.61 104.8967) (end 103.8238 104.8967) (width 0.15) (layer "F.Cu") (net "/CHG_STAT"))
 (via (at 104.277 105.3499) (size 0.45) (drill 0.2) (layers "F.Cu" "B.Cu") (capping no) (covering (front no) (back no))
  (plugging (front no) (back no)) (filling no) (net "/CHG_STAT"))
 (segment (start 110.02 106.65) (end 109.3233 106.65) (width 0.15) (layer "B.Cu") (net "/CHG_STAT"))
 (segment (start 108.0232 105.3499) (end 109.3233 106.65) (width 0.15) (layer "B.Cu") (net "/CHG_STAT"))
 (segment (start 104.277 105.3499) (end 108.0232 105.3499) (width 0.15) (layer "B.Cu") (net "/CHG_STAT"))
 (segment (start 102.4533 107.59) (end 102.31 107.4467) (width 0.15) (layer "F.Cu") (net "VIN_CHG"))
 (segment (start 102.2114 100.9033) (end 104.51 100.9033) (width 0.15) (layer "F.Cu") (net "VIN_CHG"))
 (segment (start 102.4533 108.5) (end 102.4533 107.59) (width 0.15) (layer "F.Cu") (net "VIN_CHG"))
 (segment (start 102.31 106.9) (end 102.31 107.4467) (width 0.15) (layer "F.Cu") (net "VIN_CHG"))
 (segment (start 102.0406 106.0839) (end 102.0406 101.0741) (width 0.15) (layer "F.Cu") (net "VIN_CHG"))
 (segment (start 102.0406 101.0741) (end 102.2114 100.9033) (width 0.15) (layer "F.Cu") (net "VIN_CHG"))
 (segment (start 104.51 101.7625) (end 104.51 100.9033) (width 0.15) (layer "F.Cu") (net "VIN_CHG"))
 (segment (start 102.31 106.3533) (end 102.0406 106.0839) (width 0.15) (layer "F.Cu") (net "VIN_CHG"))
 (segment (start 102.31 106.9) (end 102.31 106.3533) (width 0.15) (layer "F.Cu") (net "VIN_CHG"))
 (segment (start 102.93 108.5) (end 102.4533 108.5) (width 0.15) (layer "F.Cu") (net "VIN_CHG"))
 (segment (start 105.4067 108.46) (end 105.3667 108.5) (width 0.15) (layer "F.Cu") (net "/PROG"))
 (segment (start 104.3349 102.6217) (end 105.4067 103.6935) (width 0.15) (layer "F.Cu") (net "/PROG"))
 (segment (start 102.61 101.7625) (end 102.61 102.6217) (width 0.15) (layer "F.Cu") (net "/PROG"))
 (segment (start 105.4067 103.6935) (end 105.4067 108.46) (width 0.15) (layer "F.Cu") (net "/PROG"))
 (segment (start 102.61 102.6217) (end 104.3349 102.6217) (width 0.15) (layer "F.Cu") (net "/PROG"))
 (segment (start 104.9 108.5) (end 105.3667 108.5) (width 0.15) (layer "F.Cu") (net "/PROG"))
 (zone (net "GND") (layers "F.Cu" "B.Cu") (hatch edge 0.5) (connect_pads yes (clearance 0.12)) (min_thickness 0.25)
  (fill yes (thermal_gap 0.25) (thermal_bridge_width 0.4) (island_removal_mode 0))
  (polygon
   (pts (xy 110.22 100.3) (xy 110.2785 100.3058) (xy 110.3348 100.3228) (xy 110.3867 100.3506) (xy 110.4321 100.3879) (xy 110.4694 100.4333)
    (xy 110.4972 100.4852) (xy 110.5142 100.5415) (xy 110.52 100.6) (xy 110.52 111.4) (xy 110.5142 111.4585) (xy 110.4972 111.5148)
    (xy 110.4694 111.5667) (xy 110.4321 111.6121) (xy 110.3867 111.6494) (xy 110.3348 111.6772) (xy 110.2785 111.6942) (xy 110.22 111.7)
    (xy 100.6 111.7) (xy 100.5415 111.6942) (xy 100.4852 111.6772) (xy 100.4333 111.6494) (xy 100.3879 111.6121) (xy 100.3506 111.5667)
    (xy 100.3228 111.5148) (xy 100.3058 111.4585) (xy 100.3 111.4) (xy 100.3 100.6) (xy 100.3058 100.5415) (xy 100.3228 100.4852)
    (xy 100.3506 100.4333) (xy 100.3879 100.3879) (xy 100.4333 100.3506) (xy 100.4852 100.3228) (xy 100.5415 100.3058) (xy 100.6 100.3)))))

